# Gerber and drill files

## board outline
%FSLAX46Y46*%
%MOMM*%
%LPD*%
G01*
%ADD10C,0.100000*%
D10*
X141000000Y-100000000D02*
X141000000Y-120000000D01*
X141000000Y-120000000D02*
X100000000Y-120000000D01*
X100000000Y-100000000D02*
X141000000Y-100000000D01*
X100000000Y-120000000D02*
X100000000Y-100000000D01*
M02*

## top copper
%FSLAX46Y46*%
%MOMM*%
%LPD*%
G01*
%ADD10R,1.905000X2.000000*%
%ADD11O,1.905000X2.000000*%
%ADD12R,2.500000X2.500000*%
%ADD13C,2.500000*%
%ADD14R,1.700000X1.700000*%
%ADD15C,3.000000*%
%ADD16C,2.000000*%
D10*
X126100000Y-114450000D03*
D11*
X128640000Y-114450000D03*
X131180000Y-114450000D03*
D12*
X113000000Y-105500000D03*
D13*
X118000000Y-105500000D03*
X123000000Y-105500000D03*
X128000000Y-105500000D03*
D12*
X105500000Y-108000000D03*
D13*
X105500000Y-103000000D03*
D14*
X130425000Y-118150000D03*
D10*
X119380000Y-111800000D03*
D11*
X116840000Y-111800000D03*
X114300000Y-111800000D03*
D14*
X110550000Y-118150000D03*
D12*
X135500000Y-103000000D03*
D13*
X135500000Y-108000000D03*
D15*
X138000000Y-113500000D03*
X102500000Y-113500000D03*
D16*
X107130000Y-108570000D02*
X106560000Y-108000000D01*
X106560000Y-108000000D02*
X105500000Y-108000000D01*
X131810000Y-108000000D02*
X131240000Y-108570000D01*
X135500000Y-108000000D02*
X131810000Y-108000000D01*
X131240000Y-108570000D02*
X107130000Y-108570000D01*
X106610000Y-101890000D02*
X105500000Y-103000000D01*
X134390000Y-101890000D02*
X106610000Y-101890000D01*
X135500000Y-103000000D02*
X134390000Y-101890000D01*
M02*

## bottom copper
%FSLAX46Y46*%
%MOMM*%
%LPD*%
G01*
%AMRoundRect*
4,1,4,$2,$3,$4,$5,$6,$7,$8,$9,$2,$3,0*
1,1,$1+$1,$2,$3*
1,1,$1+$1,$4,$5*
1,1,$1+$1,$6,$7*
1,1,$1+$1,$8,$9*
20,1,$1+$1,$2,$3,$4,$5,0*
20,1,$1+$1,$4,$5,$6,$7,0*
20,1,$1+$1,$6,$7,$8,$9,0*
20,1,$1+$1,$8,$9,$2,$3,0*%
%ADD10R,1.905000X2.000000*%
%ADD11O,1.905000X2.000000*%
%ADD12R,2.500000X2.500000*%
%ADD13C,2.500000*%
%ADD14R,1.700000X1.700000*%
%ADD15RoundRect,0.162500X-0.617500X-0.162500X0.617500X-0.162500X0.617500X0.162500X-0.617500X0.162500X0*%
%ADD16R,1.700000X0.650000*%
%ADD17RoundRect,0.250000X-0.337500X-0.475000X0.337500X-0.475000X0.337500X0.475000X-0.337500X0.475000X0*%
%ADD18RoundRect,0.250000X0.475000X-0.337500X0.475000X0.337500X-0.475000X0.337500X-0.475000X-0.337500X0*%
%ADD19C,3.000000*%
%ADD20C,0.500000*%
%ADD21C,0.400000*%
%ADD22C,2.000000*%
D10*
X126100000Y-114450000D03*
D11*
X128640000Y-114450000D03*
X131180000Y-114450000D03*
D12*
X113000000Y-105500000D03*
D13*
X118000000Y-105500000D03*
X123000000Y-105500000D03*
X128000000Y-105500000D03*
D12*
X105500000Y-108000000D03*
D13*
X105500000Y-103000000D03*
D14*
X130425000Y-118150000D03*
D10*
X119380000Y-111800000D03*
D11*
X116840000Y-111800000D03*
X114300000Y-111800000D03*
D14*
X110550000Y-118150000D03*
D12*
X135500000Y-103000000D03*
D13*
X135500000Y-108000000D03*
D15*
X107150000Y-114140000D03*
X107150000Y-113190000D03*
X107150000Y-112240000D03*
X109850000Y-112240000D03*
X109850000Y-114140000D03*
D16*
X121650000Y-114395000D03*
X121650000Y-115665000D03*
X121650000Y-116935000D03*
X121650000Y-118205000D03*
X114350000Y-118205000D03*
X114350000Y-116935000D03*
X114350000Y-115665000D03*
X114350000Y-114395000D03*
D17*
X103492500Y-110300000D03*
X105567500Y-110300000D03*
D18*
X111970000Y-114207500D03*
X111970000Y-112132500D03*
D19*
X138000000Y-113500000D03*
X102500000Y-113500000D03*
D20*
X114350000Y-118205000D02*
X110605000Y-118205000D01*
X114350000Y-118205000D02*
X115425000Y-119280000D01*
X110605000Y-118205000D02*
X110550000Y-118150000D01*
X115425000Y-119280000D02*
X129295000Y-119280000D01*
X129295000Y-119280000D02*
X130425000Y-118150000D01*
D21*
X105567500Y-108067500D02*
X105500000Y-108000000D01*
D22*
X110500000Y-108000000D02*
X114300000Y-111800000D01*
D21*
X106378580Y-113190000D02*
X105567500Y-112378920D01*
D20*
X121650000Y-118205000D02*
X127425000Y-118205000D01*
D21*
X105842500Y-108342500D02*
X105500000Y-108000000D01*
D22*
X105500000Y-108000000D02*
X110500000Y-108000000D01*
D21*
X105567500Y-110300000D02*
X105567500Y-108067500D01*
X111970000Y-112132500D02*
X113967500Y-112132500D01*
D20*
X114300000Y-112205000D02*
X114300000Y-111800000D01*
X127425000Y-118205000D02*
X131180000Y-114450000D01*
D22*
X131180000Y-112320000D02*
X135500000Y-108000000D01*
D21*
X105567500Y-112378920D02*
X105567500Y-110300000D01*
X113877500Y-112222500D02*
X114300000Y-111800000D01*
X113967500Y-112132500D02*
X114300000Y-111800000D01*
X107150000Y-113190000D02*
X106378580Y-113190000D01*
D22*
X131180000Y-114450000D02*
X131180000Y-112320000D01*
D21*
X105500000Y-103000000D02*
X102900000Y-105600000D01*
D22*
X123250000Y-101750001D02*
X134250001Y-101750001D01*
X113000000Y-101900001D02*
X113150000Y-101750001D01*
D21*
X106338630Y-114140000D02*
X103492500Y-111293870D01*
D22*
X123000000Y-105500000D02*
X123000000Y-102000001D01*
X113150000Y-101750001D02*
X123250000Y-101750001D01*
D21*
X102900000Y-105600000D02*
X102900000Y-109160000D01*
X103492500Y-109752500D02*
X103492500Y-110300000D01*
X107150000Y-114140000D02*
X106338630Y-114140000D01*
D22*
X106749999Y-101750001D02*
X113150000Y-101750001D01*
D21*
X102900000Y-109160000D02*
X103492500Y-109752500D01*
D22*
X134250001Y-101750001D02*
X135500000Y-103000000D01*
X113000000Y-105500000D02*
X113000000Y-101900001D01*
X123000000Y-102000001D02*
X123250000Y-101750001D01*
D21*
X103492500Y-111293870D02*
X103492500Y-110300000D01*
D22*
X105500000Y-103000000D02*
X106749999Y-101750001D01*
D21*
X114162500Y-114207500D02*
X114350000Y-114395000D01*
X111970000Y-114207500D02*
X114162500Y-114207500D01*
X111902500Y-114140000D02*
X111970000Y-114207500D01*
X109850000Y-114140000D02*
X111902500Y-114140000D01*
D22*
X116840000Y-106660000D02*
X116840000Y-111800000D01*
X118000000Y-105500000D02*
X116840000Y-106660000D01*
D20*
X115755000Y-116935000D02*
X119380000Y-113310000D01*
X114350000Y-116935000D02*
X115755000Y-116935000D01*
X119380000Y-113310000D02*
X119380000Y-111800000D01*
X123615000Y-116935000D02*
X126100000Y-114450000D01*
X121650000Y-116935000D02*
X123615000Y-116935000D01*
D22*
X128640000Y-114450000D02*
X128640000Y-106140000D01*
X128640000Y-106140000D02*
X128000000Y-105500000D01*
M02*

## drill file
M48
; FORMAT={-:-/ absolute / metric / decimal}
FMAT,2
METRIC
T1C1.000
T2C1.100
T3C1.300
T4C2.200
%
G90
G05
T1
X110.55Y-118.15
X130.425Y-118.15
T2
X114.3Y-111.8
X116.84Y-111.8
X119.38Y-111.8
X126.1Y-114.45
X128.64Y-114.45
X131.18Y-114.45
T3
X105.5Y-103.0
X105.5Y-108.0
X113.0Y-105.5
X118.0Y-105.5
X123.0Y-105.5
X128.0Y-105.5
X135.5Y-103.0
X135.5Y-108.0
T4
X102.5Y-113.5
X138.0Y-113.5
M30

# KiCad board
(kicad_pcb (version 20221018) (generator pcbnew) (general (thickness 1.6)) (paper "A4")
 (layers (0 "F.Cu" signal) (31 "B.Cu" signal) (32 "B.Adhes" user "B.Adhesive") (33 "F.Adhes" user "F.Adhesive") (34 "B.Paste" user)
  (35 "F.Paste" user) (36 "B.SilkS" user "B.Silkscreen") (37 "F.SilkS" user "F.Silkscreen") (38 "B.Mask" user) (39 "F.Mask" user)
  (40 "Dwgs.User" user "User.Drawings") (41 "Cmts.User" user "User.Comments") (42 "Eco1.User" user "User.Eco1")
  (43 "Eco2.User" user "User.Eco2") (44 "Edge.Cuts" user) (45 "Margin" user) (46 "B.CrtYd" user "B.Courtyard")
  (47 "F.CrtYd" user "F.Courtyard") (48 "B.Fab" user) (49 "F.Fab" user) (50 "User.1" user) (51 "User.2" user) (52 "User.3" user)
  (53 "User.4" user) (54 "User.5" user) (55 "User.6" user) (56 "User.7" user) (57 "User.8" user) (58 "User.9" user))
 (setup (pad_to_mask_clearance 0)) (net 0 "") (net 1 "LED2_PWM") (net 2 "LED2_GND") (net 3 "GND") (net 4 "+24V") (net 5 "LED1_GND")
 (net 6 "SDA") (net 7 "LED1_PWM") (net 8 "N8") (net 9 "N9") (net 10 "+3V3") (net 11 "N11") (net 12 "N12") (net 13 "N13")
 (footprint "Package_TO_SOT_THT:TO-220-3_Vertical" (layer "F.Cu") (at 126.1 114.45)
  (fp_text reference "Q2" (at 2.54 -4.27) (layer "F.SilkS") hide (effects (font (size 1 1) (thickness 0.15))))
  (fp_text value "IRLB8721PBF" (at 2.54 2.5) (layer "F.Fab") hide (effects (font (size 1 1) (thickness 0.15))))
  (pad "1" thru_hole rect (at 0 0) (size 1.905 2) (drill 1.1) (layers "*.Cu" "*.Mask") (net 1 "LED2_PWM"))
  (pad "2" thru_hole oval (at 2.54 0) (size 1.905 2) (drill 1.1) (layers "*.Cu" "*.Mask") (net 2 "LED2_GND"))
  (pad "3" thru_hole oval (at 5.08 0) (size 1.905 2) (drill 1.1) (layers "*.Cu" "*.Mask") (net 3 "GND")))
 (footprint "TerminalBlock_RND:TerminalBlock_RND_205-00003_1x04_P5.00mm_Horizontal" (layer "F.Cu") (at 113 105.5)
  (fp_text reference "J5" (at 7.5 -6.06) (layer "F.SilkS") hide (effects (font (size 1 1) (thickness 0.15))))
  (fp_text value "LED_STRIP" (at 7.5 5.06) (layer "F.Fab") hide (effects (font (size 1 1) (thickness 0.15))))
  (pad "1" thru_hole rect (at 0 0) (size 2.5 2.5) (drill 1.3) (layers "*.Cu" "*.Mask") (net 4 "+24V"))
  (pad "2" thru_hole circle (at 5 0) (size 2.5 2.5) (drill 1.3) (layers "*.Cu" "*.Mask") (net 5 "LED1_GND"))
  (pad "3" thru_hole circle (at 10 0) (size 2.5 2.5) (drill 1.3) (layers "*.Cu" "*.Mask") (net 4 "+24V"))
  (pad "4" thru_hole circle (at 15 0) (size 2.5 2.5) (drill 1.3) (layers "*.Cu" "*.Mask") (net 2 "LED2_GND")))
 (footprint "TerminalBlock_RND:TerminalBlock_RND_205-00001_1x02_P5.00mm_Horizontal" (layer "F.Cu") (at 105.5 108 90)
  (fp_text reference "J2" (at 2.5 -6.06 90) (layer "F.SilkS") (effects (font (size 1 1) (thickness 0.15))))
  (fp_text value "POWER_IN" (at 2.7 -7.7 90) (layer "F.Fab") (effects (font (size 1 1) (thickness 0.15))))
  (pad "1" thru_hole rect (at 0 0 90) (size 2.5 2.5) (drill 1.3) (layers "*.Cu" "*.Mask") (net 3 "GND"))
  (pad "2" thru_hole circle (at 5 0 90) (size 2.5 2.5) (drill 1.3) (layers "*.Cu" "*.Mask") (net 4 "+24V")))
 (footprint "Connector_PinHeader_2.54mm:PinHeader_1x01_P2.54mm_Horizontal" (layer "F.Cu") (at 130.425 118.15)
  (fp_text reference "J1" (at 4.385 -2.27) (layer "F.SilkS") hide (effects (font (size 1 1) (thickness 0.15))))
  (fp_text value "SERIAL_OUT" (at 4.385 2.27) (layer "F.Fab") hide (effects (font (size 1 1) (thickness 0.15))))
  (pad "1" thru_hole rect (at 0 0) (size 1.7 1.7) (drill 1) (layers "*.Cu" "*.Mask") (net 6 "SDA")))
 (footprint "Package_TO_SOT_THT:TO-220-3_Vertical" (layer "F.Cu") (at 119.38 111.8 180)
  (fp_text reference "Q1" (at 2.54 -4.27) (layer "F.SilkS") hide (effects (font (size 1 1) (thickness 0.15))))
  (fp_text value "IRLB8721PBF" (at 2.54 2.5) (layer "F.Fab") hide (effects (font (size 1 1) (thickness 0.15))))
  (pad "1" thru_hole rect (at 0 0 180) (size 1.905 2) (drill 1.1) (layers "*.Cu" "*.Mask") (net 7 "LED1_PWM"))
  (pad "2" thru_hole oval (at 2.54 0 180) (size 1.905 2) (drill 1.1) (layers "*.Cu" "*.Mask") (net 5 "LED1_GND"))
  (pad "3" thru_hole oval (at 5.08 0 180) (size 1.905 2) (drill 1.1) (layers "*.Cu" "*.Mask") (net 3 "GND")))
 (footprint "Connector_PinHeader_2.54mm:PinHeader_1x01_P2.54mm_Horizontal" (layer "F.Cu") (at 110.55 118.15 180)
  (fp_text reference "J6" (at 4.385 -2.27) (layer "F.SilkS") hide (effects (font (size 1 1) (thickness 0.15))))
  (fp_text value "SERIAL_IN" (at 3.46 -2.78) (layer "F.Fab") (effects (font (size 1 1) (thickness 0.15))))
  (pad "1" thru_hole rect (at 0 0 180) (size 1.7 1.7) (drill 1) (layers "*.Cu" "*.Mask") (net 6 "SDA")))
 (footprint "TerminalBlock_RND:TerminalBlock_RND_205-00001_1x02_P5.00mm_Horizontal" (layer "F.Cu") (at 135.5 103 -90)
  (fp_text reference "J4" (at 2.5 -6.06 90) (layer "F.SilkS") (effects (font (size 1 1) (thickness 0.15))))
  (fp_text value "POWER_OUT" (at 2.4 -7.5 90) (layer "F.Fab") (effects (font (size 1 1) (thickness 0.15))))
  (pad "1" thru_hole rect (at 0 0 270) (size 2.5 2.5) (drill 1.3) (layers "*.Cu" "*.Mask") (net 4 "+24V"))
  (pad "2" thru_hole circle (at 5 0 270) (size 2.5 2.5) (drill 1.3) (layers "*.Cu" "*.Mask") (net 3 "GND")))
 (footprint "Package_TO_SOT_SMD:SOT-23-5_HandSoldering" (layer "B.Cu") (at 108.5 113.19)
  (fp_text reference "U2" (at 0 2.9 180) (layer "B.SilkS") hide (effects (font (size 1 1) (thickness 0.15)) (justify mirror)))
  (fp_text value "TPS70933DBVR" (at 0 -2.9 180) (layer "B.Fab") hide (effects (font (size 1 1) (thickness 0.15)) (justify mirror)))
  (pad "1" smd roundrect (at -1.35 0.95) (size 1.56 0.65) (layers "B.Cu" "B.Paste" "B.Mask") (roundrect_rratio 0.25) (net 4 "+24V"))
  (pad "2" smd roundrect (at -1.35 0) (size 1.56 0.65) (layers "B.Cu" "B.Paste" "B.Mask") (roundrect_rratio 0.25) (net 3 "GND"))
  (pad "3" smd roundrect (at -1.35 -0.95) (size 1.56 0.65) (layers "B.Cu" "B.Paste" "B.Mask") (roundrect_rratio 0.25) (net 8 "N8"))
  (pad "4" smd roundrect (at 1.35 -0.95) (size 1.56 0.65) (layers "B.Cu" "B.Paste" "B.Mask") (roundrect_rratio 0.25) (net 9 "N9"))
  (pad "5" smd roundrect (at 1.35 0.95) (size 1.56 0.65) (layers "B.Cu" "B.Paste" "B.Mask") (roundrect_rratio 0.25) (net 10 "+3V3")))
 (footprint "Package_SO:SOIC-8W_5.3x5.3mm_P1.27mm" (layer "B.Cu") (at 118 116.3 180)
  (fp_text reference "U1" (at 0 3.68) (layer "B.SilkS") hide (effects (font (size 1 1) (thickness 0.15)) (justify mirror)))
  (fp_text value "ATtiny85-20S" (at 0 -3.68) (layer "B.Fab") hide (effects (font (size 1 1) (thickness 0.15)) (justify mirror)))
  (pad "1" smd rect (at -3.65 1.905 180) (size 1.7 0.65) (layers "B.Cu" "B.Paste" "B.Mask") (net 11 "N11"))
  (pad "2" smd rect (at -3.65 0.635 180) (size 1.7 0.65) (layers "B.Cu" "B.Paste" "B.Mask") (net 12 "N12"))
  (pad "3" smd rect (at -3.65 -0.635 180) (size 1.7 0.65) (layers "B.Cu" "B.Paste" "B.Mask") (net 1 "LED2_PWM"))
  (pad "4" smd rect (at -3.65 -1.905 180) (size 1.7 0.65) (layers "B.Cu" "B.Paste" "B.Mask") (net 3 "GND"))
  (pad "5" smd rect (at 3.65 -1.905 180) (size 1.7 0.65) (layers "B.Cu" "B.Paste" "B.Mask") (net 6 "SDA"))
  (pad "6" smd rect (at 3.65 -0.635 180) (size 1.7 0.65) (layers "B.Cu" "B.Paste" "B.Mask") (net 7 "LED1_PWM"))
  (pad "7" smd rect (at 3.65 0.635 180) (size 1.7 0.65) (layers "B.Cu" "B.Paste" "B.Mask") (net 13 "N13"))
  (pad "8" smd rect (at 3.65 1.905 180) (size 1.7 0.65) (layers "B.Cu" "B.Paste" "B.Mask") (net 10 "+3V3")))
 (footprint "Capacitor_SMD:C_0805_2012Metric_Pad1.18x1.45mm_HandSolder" (layer "B.Cu") (at 104.53 110.3)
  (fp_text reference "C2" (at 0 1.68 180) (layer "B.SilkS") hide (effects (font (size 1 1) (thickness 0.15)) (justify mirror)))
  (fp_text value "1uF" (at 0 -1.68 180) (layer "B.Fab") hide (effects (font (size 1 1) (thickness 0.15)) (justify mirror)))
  (pad "1" smd roundrect (at -1.0375 0) (size 1.175 1.45) (layers "B.Cu" "B.Paste" "B.Mask") (roundrect_rratio 0.212766) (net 4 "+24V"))
  (pad "2" smd roundrect (at 1.0375 0) (size 1.175 1.45) (layers "B.Cu" "B.Paste" "B.Mask") (roundrect_rratio 0.212766) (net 3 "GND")))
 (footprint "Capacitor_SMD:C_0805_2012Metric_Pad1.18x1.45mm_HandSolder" (layer "B.Cu") (at 111.97 113.17 90)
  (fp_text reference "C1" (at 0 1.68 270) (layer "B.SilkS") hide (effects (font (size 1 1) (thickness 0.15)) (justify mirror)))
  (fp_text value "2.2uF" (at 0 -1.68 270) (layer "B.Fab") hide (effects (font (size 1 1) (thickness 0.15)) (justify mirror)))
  (pad "1" smd roundrect (at -1.0375 0 90) (size 1.175 1.45) (layers "B.Cu" "B.Paste" "B.Mask") (roundrect_rratio 0.212766) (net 10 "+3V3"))
  (pad "2" smd roundrect (at 1.0375 0 90) (size 1.175 1.45) (layers "B.Cu" "B.Paste" "B.Mask") (roundrect_rratio 0.212766) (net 3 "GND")))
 (gr_line (start 141 100) (end 141 120) (stroke (width 0.1) (type default)) (layer "Edge.Cuts"))
 (gr_line (start 141 120) (end 100 120) (stroke (width 0.1) (type default)) (layer "Edge.Cuts"))
 (gr_line (start 100 100) (end 141 100) (stroke (width 0.1) (type default)) (layer "Edge.Cuts"))
 (gr_line (start 100 120) (end 100 100) (stroke (width 0.1) (type default)) (layer "Edge.Cuts"))
 (via (at 138 113.5) (size 3) (drill 2.2) (layers "F.Cu" "B.Cu") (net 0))
 (via (at 102.5 113.5) (size 3) (drill 2.2) (layers "F.Cu" "B.Cu") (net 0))
 (segment (start 114.35 118.205) (end 110.605 118.205) (width 0.5) (layer "B.Cu") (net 6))
 (segment (start 114.35 118.205) (end 115.425 119.28) (width 0.5) (layer "B.Cu") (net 6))
 (segment (start 110.605 118.205) (end 110.55 118.15) (width 0.5) (layer "B.Cu") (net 6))
 (segment (start 115.425 119.28) (end 129.295 119.28) (width 0.5) (layer "B.Cu") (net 6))
 (segment (start 129.295 119.28) (end 130.425 118.15) (width 0.5) (layer "B.Cu") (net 6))
 (segment (start 107.13 108.57) (end 106.56 108) (width 2) (layer "F.Cu") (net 3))
 (segment (start 106.56 108) (end 105.5 108) (width 2) (layer "F.Cu") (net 3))
 (segment (start 131.81 108) (end 131.24 108.57) (width 2) (layer "F.Cu") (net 3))
 (segment (start 135.5 108) (end 131.81 108) (width 2) (layer "F.Cu") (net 3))
 (segment (start 131.24 108.57) (end 107.13 108.57) (width 2) (layer "F.Cu") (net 3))
 (segment (start 105.5675 108.0675) (end 105.5 108) (width 0.4) (layer "B.Cu") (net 3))
 (segment (start 110.5 108) (end 114.3 111.8) (width 2) (layer "B.Cu") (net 3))
 (segment (start 106.37858 113.19) (end 105.5675 112.37892) (width 0.4) (layer "B.Cu") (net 3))
 (segment (start 121.65 118.205) (end 127.425 118.205) (width 0.5) (layer "B.Cu") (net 3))
 (segment (start 105.8425 108.3425) (end 105.5 108) (width 0.4) (layer "B.Cu") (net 3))
 (segment (start 105.5 108) (end 110.5 108) (width 2) (layer "B.Cu") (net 3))
 (segment (start 105.5675 110.3) (end 105.5675 108.0675) (width 0.4) (layer "B.Cu") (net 3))
 (segment (start 111.97 112.1325) (end 113.9675 112.1325) (width 0.4) (layer "B.Cu") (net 3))
 (segment (start 114.3 112.205) (end 114.3 111.8) (width 0.5) (layer "B.Cu") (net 3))
 (segment (start 127.425 118.205) (end 131.18 114.45) (width 0.5) (layer "B.Cu") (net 3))
 (segment (start 131.18 112.32) (end 135.5 108) (width 2) (layer "B.Cu") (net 3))
 (segment (start 105.5675 112.37892) (end 105.5675 110.3) (width 0.4) (layer "B.Cu") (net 3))
 (segment (start 113.8775 112.2225) (end 114.3 111.8) (width 0.4) (layer "B.Cu") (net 3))
 (segment (start 113.9675 112.1325) (end 114.3 111.8) (width 0.4) (layer "B.Cu") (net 3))
 (segment (start 107.15 113.19) (end 106.37858 113.19) (width 0.4) (layer "B.Cu") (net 3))
 (segment (start 131.18 114.45) (end 131.18 112.32) (width 2) (layer "B.Cu") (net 3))
 (segment (start 106.61 101.89) (end 105.5 103) (width 2) (layer "F.Cu") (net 4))
 (segment (start 134.39 101.89) (end 106.61 101.89) (width 2) (layer "F.Cu") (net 4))
 (segment (start 135.5 103) (end 134.39 101.89) (width 2) (layer "F.Cu") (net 4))
 (segment (start 105.5 103) (end 102.9 105.6) (width 0.4) (layer "B.Cu") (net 4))
 (segment (start 123.25 101.750001) (end 134.250001 101.750001) (width 2) (layer "B.Cu") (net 4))
 (segment (start 113 101.900001) (end 113.15 101.750001) (width 2) (layer "B.Cu") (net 4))
 (segment (start 106.33863 114.14) (end 103.4925 111.29387) (width 0.4) (layer "B.Cu") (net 4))
 (segment (start 123 105.5) (end 123 102.000001) (width 2) (layer "B.Cu") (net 4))
 (segment (start 113.15 101.750001) (end 123.25 101.750001) (width 2) (layer "B.Cu") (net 4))
 (segment (start 102.9 105.6) (end 102.9 109.16) (width 0.4) (layer "B.Cu") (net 4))
 (segment (start 103.4925 109.7525) (end 103.4925 110.3) (width 0.4) (layer "B.Cu") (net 4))
 (segment (start 107.15 114.14) (end 106.33863 114.14) (width 0.4) (layer "B.Cu") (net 4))
 (segment (start 106.749999 101.750001) (end 113.15 101.750001) (width 2) (layer "B.Cu") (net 4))
 (segment (start 102.9 109.16) (end 103.4925 109.7525) (width 0.4) (layer "B.Cu") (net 4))
 (segment (start 134.250001 101.750001) (end 135.5 103) (width 2) (layer "B.Cu") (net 4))
 (segment (start 113 105.5) (end 113 101.900001) (width 2) (layer "B.Cu") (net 4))
 (segment (start 123 102.000001) (end 123.25 101.750001) (width 2) (layer "B.Cu") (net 4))
 (segment (start 103.4925 111.29387) (end 103.4925 110.3) (width 0.4) (layer "B.Cu") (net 4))
 (segment (start 105.5 103) (end 106.749999 101.750001) (width 2) (layer "B.Cu") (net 4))
 (segment (start 114.1625 114.2075) (end 114.35 114.395) (width 0.4) (layer "B.Cu") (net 10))
 (segment (start 111.97 114.2075) (end 114.1625 114.2075) (width 0.4) (layer "B.Cu") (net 10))
 (segment (start 111.9025 114.14) (end 111.97 114.2075) (width 0.4) (layer "B.Cu") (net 10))
 (segment (start 109.85 114.14) (end 111.9025 114.14) (width 0.4) (layer "B.Cu") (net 10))
 (segment (start 116.84 106.66) (end 116.84 111.8) (width 2) (layer "B.Cu") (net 5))
 (segment (start 118 105.5) (end 116.84 106.66) (width 2) (layer "B.Cu") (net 5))
 (segment (start 115.755 116.935) (end 119.38 113.31) (width 0.5) (layer "B.Cu") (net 7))
 (segment (start 114.35 116.935) (end 115.755 116.935) (width 0.5) (layer "B.Cu") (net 7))
 (segment (start 119.38 113.31) (end 119.38 111.8) (width 0.5) (layer "B.Cu") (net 7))
 (segment (start 123.615 116.935) (end 126.1 114.45) (width 0.5) (layer "B.Cu") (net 1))
 (segment (start 121.65 116.935) (end 123.615 116.935) (width 0.5) (layer "B.Cu") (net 1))
 (segment (start 128.64 114.45) (end 128.64 106.14) (width 2) (layer "B.Cu") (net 2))
 (segment (start 128.64 106.14) (end 128 105.5) (width 2) (layer "B.Cu") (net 2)))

